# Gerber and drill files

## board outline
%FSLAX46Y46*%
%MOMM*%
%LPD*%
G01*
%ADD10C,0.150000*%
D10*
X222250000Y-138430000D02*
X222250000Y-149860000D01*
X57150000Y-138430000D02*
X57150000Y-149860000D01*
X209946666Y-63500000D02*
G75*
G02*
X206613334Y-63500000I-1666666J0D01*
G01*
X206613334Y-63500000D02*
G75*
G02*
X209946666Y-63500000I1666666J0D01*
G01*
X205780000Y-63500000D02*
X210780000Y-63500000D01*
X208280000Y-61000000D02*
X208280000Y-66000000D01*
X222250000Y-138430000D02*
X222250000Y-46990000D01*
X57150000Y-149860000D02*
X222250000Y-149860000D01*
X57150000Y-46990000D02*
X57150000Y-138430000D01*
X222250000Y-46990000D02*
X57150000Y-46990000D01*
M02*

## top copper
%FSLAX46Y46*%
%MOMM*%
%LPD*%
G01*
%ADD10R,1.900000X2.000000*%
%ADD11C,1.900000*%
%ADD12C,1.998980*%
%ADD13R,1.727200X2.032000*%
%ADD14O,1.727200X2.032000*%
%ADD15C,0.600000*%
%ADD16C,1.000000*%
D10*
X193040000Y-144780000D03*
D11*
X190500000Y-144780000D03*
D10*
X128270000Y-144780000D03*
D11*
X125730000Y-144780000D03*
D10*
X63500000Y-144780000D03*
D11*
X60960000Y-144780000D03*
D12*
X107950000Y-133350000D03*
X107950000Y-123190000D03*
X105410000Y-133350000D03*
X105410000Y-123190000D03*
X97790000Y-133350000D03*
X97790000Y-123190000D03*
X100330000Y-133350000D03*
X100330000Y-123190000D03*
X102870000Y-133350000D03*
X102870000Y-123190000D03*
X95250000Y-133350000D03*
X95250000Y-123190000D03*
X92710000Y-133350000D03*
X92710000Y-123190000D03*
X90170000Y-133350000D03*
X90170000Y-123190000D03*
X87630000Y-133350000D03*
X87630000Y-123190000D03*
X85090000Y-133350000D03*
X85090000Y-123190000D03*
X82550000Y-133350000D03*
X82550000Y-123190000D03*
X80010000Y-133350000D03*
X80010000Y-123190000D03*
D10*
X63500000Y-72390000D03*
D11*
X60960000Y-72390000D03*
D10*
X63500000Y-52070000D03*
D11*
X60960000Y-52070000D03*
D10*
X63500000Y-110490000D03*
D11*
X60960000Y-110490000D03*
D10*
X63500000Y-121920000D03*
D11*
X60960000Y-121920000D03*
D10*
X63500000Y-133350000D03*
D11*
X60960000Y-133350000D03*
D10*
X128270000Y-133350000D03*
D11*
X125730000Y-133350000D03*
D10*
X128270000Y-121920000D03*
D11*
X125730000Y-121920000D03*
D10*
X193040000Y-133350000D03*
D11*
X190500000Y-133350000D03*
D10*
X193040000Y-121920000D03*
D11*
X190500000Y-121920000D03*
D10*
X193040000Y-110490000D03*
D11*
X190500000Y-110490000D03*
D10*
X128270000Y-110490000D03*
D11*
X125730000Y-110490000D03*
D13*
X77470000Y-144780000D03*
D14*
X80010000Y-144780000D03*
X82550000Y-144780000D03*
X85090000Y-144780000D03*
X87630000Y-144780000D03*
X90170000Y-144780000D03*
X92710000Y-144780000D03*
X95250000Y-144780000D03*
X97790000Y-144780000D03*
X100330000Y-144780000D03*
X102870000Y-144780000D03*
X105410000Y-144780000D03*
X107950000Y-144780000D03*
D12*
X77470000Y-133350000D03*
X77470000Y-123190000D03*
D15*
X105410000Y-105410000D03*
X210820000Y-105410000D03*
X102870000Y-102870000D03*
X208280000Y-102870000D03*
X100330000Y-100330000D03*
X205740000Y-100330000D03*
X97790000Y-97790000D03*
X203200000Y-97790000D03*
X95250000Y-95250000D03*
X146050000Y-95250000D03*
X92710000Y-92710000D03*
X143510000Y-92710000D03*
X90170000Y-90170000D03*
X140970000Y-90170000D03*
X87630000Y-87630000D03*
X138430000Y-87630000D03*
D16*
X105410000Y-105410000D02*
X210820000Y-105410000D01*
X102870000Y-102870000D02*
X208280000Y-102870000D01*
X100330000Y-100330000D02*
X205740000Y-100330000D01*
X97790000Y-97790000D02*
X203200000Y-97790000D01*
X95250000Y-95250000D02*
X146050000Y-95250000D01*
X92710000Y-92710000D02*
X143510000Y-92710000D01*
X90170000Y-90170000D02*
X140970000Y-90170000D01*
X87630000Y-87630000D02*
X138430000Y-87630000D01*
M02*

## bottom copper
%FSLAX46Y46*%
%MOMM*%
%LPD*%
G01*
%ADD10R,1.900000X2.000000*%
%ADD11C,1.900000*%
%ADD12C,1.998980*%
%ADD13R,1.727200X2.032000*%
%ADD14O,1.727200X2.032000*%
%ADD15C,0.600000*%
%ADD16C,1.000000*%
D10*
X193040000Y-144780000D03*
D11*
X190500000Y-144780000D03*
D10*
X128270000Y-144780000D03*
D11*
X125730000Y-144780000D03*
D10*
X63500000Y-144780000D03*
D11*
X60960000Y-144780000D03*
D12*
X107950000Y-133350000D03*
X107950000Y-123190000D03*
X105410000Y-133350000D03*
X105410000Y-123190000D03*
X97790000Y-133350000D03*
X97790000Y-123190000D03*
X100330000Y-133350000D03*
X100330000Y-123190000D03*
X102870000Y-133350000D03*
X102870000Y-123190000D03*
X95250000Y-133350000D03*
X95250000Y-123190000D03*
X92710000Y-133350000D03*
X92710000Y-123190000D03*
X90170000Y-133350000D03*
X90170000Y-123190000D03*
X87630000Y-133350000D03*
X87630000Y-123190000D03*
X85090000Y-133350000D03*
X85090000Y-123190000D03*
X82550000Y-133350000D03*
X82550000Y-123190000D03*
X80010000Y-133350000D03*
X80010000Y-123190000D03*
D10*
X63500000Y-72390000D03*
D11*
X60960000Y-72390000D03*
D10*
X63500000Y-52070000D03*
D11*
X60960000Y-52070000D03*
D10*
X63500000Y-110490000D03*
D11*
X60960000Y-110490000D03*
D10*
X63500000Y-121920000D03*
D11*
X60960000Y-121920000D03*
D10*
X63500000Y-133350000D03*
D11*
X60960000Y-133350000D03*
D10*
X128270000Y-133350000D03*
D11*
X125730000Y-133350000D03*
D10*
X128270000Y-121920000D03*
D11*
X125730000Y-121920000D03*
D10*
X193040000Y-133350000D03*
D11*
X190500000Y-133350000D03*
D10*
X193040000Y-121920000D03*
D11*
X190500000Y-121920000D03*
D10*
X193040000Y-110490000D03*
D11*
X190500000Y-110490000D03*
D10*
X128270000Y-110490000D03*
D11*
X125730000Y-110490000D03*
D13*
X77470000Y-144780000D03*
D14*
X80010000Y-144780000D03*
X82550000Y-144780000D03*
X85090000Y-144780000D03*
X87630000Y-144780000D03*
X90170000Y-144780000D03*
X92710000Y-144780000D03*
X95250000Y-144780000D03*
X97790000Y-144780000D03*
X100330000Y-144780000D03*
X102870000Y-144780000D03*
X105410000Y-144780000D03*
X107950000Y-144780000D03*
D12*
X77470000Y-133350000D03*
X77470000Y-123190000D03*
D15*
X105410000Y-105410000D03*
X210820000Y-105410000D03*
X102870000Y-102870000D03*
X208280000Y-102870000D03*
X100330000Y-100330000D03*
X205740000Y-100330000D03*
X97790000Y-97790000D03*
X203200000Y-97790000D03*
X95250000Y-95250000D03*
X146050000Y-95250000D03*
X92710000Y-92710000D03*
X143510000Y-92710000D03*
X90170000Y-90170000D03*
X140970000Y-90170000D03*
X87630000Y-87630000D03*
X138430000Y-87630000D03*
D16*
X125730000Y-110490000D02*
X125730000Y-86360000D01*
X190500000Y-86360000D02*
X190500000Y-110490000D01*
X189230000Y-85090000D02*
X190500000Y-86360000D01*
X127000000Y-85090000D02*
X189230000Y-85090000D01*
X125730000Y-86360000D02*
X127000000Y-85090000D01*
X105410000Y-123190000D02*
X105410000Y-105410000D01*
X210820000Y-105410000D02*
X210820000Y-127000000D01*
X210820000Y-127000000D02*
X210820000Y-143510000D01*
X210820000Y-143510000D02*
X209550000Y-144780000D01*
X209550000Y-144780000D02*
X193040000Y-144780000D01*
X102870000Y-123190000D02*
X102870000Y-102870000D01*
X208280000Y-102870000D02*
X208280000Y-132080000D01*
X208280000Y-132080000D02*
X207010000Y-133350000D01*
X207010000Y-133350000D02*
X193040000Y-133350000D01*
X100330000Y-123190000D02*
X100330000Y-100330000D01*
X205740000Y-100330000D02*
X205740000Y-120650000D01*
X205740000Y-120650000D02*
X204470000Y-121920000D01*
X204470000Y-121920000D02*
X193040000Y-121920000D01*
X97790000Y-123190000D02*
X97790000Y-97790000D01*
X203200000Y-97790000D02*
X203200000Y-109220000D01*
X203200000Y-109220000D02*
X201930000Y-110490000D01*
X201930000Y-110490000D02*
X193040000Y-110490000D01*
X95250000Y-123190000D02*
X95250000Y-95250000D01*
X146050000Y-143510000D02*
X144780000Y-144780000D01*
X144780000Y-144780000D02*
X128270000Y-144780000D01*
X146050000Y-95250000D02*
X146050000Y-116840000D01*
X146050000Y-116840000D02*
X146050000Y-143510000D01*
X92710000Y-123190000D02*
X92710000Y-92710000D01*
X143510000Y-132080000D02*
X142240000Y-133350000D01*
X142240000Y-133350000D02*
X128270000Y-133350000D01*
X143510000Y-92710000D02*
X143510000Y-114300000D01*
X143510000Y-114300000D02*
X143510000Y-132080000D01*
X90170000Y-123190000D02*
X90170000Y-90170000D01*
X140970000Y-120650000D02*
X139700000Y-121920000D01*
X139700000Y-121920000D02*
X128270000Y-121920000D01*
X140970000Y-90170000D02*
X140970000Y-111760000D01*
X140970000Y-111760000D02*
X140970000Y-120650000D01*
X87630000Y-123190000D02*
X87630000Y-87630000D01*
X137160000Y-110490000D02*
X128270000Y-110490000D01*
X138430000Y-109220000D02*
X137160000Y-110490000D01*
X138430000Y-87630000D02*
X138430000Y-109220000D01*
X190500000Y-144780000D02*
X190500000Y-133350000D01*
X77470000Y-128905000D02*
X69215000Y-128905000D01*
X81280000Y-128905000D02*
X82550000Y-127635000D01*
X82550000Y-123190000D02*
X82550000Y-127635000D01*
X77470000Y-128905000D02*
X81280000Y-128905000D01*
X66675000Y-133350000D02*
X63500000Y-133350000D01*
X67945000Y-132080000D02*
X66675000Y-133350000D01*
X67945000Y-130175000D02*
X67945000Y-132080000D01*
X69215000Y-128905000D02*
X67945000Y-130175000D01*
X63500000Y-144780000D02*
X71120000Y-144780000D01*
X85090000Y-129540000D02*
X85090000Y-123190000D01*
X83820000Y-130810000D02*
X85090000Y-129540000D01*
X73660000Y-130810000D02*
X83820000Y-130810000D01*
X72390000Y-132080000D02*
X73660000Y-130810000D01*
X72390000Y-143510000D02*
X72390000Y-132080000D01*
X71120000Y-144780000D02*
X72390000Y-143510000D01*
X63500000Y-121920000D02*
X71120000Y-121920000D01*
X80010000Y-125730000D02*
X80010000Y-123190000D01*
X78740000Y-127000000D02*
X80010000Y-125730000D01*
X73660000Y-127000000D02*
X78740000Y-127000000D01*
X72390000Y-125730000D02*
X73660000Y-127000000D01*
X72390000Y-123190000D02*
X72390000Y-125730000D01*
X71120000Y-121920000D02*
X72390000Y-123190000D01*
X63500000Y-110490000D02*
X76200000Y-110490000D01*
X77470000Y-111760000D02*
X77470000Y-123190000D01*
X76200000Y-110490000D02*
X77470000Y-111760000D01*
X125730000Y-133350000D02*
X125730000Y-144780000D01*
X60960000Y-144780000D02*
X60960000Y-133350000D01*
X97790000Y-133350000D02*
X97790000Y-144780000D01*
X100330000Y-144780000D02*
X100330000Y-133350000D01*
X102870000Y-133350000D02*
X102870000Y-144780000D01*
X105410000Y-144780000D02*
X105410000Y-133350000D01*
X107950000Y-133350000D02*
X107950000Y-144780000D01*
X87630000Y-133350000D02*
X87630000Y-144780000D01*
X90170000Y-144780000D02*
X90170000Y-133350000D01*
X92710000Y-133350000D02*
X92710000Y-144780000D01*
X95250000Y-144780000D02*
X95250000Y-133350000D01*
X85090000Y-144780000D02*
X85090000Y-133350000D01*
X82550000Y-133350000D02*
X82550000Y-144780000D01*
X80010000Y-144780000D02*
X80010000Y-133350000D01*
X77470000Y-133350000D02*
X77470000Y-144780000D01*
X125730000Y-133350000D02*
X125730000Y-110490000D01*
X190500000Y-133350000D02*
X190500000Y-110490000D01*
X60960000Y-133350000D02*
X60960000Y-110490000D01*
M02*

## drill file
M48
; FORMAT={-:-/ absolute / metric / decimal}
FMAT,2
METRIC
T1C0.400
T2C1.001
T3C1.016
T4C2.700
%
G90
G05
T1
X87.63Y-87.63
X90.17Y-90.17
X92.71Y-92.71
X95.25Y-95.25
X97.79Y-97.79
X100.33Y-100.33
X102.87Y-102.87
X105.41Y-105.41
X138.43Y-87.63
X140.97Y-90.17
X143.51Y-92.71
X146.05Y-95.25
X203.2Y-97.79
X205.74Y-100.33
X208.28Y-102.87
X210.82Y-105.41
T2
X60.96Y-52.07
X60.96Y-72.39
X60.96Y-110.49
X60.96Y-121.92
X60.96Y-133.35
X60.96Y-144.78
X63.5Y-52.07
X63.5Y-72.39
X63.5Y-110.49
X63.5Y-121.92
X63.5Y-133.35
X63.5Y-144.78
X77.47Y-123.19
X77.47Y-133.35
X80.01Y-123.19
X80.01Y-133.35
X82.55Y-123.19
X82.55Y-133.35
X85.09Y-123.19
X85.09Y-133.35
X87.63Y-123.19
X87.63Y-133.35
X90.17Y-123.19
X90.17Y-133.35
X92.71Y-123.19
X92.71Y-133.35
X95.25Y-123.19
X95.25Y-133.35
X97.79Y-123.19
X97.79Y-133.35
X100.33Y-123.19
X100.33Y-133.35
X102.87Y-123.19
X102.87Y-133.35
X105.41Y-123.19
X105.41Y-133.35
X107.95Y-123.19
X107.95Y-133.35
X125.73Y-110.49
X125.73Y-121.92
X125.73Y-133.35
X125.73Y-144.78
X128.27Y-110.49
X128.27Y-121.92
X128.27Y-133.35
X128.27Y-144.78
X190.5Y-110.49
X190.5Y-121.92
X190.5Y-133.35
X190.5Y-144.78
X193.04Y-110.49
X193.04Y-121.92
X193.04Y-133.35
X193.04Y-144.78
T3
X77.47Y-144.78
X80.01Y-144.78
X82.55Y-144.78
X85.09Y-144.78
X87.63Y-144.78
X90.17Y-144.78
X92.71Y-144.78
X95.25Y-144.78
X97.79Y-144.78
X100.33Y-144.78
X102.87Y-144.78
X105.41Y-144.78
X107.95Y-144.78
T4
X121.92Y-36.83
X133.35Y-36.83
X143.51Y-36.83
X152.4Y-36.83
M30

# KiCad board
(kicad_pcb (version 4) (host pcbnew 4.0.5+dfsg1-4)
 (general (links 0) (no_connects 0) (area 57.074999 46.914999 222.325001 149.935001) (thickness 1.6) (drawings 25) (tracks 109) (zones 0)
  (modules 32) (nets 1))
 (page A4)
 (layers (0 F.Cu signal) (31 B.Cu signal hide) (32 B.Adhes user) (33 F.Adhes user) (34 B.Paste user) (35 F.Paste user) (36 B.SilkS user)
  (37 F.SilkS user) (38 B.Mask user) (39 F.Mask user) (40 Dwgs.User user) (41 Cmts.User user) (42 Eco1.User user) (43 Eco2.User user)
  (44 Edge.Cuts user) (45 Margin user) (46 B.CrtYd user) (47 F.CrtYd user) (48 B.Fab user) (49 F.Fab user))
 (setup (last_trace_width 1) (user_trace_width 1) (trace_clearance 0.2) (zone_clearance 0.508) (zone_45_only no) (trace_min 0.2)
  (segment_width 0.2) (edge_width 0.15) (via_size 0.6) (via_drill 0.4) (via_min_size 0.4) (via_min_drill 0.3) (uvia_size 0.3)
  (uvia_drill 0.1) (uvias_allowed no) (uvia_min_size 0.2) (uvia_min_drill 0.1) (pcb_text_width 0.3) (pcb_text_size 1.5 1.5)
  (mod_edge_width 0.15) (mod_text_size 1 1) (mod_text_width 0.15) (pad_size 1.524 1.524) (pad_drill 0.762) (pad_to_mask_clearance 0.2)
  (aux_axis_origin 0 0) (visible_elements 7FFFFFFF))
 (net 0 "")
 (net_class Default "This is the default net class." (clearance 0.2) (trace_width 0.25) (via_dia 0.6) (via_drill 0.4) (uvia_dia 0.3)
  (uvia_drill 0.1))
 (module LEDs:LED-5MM (layer F.Cu) (at 193.04 144.78 180)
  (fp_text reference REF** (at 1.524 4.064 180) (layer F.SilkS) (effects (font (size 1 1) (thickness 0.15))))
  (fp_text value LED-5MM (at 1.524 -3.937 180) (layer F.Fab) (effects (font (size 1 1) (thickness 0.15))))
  (pad 1 thru_hole rect (at 0 0 270) (size 2 1.9) (drill 1.00076) (layers *.Cu *.Mask))
  (pad 2 thru_hole circle (at 2.54 0 180) (size 1.9 1.9) (drill 1.00076) (layers *.Cu *.Mask)))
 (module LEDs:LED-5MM (layer F.Cu) (at 128.27 144.78 180)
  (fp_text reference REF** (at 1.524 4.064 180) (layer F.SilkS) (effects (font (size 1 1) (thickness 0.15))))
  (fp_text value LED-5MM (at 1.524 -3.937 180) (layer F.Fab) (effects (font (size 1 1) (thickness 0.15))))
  (pad 1 thru_hole rect (at 0 0 270) (size 2 1.9) (drill 1.00076) (layers *.Cu *.Mask))
  (pad 2 thru_hole circle (at 2.54 0 180) (size 1.9 1.9) (drill 1.00076) (layers *.Cu *.Mask)))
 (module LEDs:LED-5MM (layer F.Cu) (at 63.5 144.78 180)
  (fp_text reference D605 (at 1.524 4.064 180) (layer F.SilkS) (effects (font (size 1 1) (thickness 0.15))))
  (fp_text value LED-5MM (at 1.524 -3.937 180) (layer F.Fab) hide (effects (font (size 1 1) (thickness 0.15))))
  (pad 1 thru_hole rect (at 0 0 270) (size 2 1.9) (drill 1.00076) (layers *.Cu *.Mask))
  (pad 2 thru_hole circle (at 2.54 0 180) (size 1.9 1.9) (drill 1.00076) (layers *.Cu *.Mask)))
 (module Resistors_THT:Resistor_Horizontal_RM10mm (layer F.Cu) (at 107.95 133.35 90)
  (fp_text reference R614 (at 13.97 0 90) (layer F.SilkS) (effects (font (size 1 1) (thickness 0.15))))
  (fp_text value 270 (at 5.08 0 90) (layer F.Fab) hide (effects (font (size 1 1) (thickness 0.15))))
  (pad 1 thru_hole circle (at 0 0 90) (size 1.99898 1.99898) (drill 1.00076) (layers *.Cu *.SilkS *.Mask))
  (pad 2 thru_hole circle (at 10.16 0 90) (size 1.99898 1.99898) (drill 1.00076) (layers *.Cu *.SilkS *.Mask)))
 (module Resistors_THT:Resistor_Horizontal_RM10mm (layer F.Cu) (at 105.41 133.35 90)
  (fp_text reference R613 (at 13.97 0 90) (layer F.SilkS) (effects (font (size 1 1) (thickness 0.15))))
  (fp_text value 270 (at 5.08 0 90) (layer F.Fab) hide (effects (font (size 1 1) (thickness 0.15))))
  (pad 1 thru_hole circle (at 0 0 90) (size 1.99898 1.99898) (drill 1.00076) (layers *.Cu *.SilkS *.Mask))
  (pad 2 thru_hole circle (at 10.16 0 90) (size 1.99898 1.99898) (drill 1.00076) (layers *.Cu *.SilkS *.Mask)))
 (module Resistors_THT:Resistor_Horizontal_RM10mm (layer F.Cu) (at 97.79 133.35 90)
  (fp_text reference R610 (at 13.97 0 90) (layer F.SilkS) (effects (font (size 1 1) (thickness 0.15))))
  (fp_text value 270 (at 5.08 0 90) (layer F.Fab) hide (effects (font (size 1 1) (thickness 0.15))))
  (pad 1 thru_hole circle (at 0 0 90) (size 1.99898 1.99898) (drill 1.00076) (layers *.Cu *.SilkS *.Mask))
  (pad 2 thru_hole circle (at 10.16 0 90) (size 1.99898 1.99898) (drill 1.00076) (layers *.Cu *.SilkS *.Mask)))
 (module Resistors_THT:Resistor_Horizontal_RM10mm (layer F.Cu) (at 100.33 133.35 90)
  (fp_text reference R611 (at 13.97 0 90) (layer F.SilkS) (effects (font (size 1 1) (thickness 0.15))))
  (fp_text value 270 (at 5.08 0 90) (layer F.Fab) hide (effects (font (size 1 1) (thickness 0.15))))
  (pad 1 thru_hole circle (at 0 0 90) (size 1.99898 1.99898) (drill 1.00076) (layers *.Cu *.SilkS *.Mask))
  (pad 2 thru_hole circle (at 10.16 0 90) (size 1.99898 1.99898) (drill 1.00076) (layers *.Cu *.SilkS *.Mask)))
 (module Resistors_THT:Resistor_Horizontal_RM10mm (layer F.Cu) (at 102.87 133.35 90)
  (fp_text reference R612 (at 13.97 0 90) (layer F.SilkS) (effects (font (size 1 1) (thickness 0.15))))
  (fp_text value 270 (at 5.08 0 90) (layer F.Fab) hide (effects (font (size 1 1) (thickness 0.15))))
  (pad 1 thru_hole circle (at 0 0 90) (size 1.99898 1.99898) (drill 1.00076) (layers *.Cu *.SilkS *.Mask))
  (pad 2 thru_hole circle (at 10.16 0 90) (size 1.99898 1.99898) (drill 1.00076) (layers *.Cu *.SilkS *.Mask)))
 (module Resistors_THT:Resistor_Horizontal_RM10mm (layer F.Cu) (at 95.25 133.35 90)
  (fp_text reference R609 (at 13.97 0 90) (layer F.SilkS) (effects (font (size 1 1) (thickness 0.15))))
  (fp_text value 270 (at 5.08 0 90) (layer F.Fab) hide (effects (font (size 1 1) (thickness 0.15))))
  (pad 1 thru_hole circle (at 0 0 90) (size 1.99898 1.99898) (drill 1.00076) (layers *.Cu *.SilkS *.Mask))
  (pad 2 thru_hole circle (at 10.16 0 90) (size 1.99898 1.99898) (drill 1.00076) (layers *.Cu *.SilkS *.Mask)))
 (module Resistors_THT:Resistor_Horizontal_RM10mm (layer F.Cu) (at 92.71 133.35 90)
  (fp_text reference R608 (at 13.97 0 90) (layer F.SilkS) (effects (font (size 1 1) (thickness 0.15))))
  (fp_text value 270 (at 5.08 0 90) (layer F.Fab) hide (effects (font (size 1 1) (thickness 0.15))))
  (pad 1 thru_hole circle (at 0 0 90) (size 1.99898 1.99898) (drill 1.00076) (layers *.Cu *.SilkS *.Mask))
  (pad 2 thru_hole circle (at 10.16 0 90) (size 1.99898 1.99898) (drill 1.00076) (layers *.Cu *.SilkS *.Mask)))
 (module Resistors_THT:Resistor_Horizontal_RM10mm (layer F.Cu) (at 90.17 133.35 90)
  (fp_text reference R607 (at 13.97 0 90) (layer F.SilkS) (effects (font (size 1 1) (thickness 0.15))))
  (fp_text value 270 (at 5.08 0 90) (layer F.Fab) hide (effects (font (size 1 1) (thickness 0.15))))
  (pad 1 thru_hole circle (at 0 0 90) (size 1.99898 1.99898) (drill 1.00076) (layers *.Cu *.SilkS *.Mask))
  (pad 2 thru_hole circle (at 10.16 0 90) (size 1.99898 1.99898) (drill 1.00076) (layers *.Cu *.SilkS *.Mask)))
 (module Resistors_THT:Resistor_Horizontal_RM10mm (layer F.Cu) (at 87.63 133.35 90)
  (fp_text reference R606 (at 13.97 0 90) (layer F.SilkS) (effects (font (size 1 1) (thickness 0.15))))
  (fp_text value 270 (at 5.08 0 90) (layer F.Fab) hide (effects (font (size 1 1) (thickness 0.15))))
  (pad 1 thru_hole circle (at 0 0 90) (size 1.99898 1.99898) (drill 1.00076) (layers *.Cu *.SilkS *.Mask))
  (pad 2 thru_hole circle (at 10.16 0 90) (size 1.99898 1.99898) (drill 1.00076) (layers *.Cu *.SilkS *.Mask)))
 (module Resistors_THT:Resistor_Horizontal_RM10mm (layer F.Cu) (at 85.09 133.35 90)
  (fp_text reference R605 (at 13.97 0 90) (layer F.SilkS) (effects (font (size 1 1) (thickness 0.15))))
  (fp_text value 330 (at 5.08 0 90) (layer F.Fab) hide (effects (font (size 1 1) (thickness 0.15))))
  (pad 1 thru_hole circle (at 0 0 90) (size 1.99898 1.99898) (drill 1.00076) (layers *.Cu *.SilkS *.Mask))
  (pad 2 thru_hole circle (at 10.16 0 90) (size 1.99898 1.99898) (drill 1.00076) (layers *.Cu *.SilkS *.Mask)))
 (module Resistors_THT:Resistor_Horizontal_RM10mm (layer F.Cu) (at 82.55 133.35 90)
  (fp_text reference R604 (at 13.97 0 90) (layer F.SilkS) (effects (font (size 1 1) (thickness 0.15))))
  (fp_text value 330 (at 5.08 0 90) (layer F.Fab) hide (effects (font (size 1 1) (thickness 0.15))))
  (pad 1 thru_hole circle (at 0 0 90) (size 1.99898 1.99898) (drill 1.00076) (layers *.Cu *.SilkS *.Mask))
  (pad 2 thru_hole circle (at 10.16 0 90) (size 1.99898 1.99898) (drill 1.00076) (layers *.Cu *.SilkS *.Mask)))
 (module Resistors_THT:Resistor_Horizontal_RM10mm (layer F.Cu) (at 80.01 133.35 90)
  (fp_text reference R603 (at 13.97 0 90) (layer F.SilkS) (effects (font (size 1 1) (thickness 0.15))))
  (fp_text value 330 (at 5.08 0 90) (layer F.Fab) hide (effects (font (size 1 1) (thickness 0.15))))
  (pad 1 thru_hole circle (at 0 0 90) (size 1.99898 1.99898) (drill 1.00076) (layers *.Cu *.SilkS *.Mask))
  (pad 2 thru_hole circle (at 10.16 0 90) (size 1.99898 1.99898) (drill 1.00076) (layers *.Cu *.SilkS *.Mask)))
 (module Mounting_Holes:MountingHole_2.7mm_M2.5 (layer F.Cu) (at 152.4 36.83)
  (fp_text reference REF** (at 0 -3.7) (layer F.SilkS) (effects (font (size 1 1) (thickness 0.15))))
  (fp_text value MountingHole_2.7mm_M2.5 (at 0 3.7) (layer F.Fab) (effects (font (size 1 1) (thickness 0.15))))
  (pad 1 np_thru_hole circle (at 0 0) (size 2.7 2.7) (drill 2.7) (layers *.Cu *.Mask)))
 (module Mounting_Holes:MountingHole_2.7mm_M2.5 (layer F.Cu) (at 143.51 36.83)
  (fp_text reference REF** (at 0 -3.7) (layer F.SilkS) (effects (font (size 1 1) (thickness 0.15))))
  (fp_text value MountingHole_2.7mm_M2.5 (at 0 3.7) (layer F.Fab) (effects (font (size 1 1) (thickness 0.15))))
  (pad 1 np_thru_hole circle (at 0 0) (size 2.7 2.7) (drill 2.7) (layers *.Cu *.Mask)))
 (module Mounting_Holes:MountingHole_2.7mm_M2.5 (layer F.Cu) (at 133.35 36.83)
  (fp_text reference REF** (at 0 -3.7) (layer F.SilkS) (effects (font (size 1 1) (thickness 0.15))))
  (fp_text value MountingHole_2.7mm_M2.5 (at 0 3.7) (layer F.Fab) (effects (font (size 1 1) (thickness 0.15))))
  (pad 1 np_thru_hole circle (at 0 0) (size 2.7 2.7) (drill 2.7) (layers *.Cu *.Mask)))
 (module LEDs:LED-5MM (layer F.Cu) (at 63.5 72.39 180)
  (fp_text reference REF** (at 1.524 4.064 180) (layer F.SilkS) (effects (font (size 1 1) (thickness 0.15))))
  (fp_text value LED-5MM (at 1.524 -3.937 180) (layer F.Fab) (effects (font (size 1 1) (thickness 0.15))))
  (pad 1 thru_hole rect (at 0 0 270) (size 2 1.9) (drill 1.00076) (layers *.Cu *.Mask))
  (pad 2 thru_hole circle (at 2.54 0 180) (size 1.9 1.9) (drill 1.00076) (layers *.Cu *.Mask)))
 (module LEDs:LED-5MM (layer F.Cu) (at 63.5 52.07 180)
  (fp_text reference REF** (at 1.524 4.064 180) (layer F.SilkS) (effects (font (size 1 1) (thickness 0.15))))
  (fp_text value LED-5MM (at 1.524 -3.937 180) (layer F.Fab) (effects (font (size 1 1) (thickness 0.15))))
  (pad 1 thru_hole rect (at 0 0 270) (size 2 1.9) (drill 1.00076) (layers *.Cu *.Mask))
  (pad 2 thru_hole circle (at 2.54 0 180) (size 1.9 1.9) (drill 1.00076) (layers *.Cu *.Mask)))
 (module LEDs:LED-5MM (layer F.Cu) (at 63.5 110.49 180)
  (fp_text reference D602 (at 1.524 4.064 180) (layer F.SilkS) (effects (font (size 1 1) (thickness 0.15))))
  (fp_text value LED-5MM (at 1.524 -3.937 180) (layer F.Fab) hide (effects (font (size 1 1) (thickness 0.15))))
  (pad 1 thru_hole rect (at 0 0 270) (size 2 1.9) (drill 1.00076) (layers *.Cu *.Mask))
  (pad 2 thru_hole circle (at 2.54 0 180) (size 1.9 1.9) (drill 1.00076) (layers *.Cu *.Mask)))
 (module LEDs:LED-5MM (layer F.Cu) (at 63.5 121.92 180)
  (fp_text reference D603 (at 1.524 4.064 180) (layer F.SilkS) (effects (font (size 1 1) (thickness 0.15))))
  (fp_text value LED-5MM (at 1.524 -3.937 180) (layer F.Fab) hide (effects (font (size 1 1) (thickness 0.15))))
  (pad 1 thru_hole rect (at 0 0 270) (size 2 1.9) (drill 1.00076) (layers *.Cu *.Mask))
  (pad 2 thru_hole circle (at 2.54 0 180) (size 1.9 1.9) (drill 1.00076) (layers *.Cu *.Mask)))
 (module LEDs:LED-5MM (layer F.Cu) (at 63.5 133.35 180)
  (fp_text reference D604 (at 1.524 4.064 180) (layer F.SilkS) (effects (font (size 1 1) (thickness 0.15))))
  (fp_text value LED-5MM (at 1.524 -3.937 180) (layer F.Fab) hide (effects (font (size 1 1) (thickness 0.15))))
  (pad 1 thru_hole rect (at 0 0 270) (size 2 1.9) (drill 1.00076) (layers *.Cu *.Mask))
  (pad 2 thru_hole circle (at 2.54 0 180) (size 1.9 1.9) (drill 1.00076) (layers *.Cu *.Mask)))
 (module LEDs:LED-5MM (layer F.Cu) (at 128.27 133.35 180)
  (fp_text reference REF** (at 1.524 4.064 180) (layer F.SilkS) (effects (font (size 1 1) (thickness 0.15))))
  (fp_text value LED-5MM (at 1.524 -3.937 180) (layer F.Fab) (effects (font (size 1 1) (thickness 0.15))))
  (pad 1 thru_hole rect (at 0 0 270) (size 2 1.9) (drill 1.00076) (layers *.Cu *.Mask))
  (pad 2 thru_hole circle (at 2.54 0 180) (size 1.9 1.9) (drill 1.00076) (layers *.Cu *.Mask)))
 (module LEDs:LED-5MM (layer F.Cu) (at 128.27 121.92 180)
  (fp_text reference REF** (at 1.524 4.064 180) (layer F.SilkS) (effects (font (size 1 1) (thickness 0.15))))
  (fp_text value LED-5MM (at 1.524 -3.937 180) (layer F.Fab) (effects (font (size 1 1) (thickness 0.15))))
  (pad 1 thru_hole rect (at 0 0 270) (size 2 1.9) (drill 1.00076) (layers *.Cu *.Mask))
  (pad 2 thru_hole circle (at 2.54 0 180) (size 1.9 1.9) (drill 1.00076) (layers *.Cu *.Mask)))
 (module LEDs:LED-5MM (layer F.Cu) (at 193.04 133.35 180)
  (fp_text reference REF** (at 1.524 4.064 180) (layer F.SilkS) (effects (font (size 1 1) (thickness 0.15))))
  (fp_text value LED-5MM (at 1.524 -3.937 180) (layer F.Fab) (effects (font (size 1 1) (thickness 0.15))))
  (pad 1 thru_hole rect (at 0 0 270) (size 2 1.9) (drill 1.00076) (layers *.Cu *.Mask))
  (pad 2 thru_hole circle (at 2.54 0 180) (size 1.9 1.9) (drill 1.00076) (layers *.Cu *.Mask)))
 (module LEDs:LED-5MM (layer F.Cu) (at 193.04 121.92 180)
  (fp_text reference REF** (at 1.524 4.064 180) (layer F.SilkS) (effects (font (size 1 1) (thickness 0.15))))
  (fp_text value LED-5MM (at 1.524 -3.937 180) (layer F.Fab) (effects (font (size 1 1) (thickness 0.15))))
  (pad 1 thru_hole rect (at 0 0 270) (size 2 1.9) (drill 1.00076) (layers *.Cu *.Mask))
  (pad 2 thru_hole circle (at 2.54 0 180) (size 1.9 1.9) (drill 1.00076) (layers *.Cu *.Mask)))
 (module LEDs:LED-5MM (layer F.Cu) (at 193.04 110.49 180)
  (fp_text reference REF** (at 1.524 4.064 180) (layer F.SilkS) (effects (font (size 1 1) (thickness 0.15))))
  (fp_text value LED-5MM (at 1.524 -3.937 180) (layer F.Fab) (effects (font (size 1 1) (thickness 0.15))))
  (pad 1 thru_hole rect (at 0 0 270) (size 2 1.9) (drill 1.00076) (layers *.Cu *.Mask))
  (pad 2 thru_hole circle (at 2.54 0 180) (size 1.9 1.9) (drill 1.00076) (layers *.Cu *.Mask)))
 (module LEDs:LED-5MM (layer F.Cu) (at 128.27 110.49 180)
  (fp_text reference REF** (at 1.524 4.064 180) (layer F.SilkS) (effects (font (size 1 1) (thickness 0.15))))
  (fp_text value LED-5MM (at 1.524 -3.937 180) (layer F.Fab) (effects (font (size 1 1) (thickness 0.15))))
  (pad 1 thru_hole rect (at 0 0 270) (size 2 1.9) (drill 1.00076) (layers *.Cu *.Mask))
  (pad 2 thru_hole circle (at 2.54 0 180) (size 1.9 1.9) (drill 1.00076) (layers *.Cu *.Mask)))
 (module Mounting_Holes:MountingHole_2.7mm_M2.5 (layer F.Cu) (at 121.92 36.83)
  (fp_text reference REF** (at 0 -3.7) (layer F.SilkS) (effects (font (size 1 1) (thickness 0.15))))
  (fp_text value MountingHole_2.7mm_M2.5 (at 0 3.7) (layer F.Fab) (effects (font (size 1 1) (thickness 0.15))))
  (pad 1 np_thru_hole circle (at 0 0) (size 2.7 2.7) (drill 2.7) (layers *.Cu *.Mask)))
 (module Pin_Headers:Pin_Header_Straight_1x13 (layer F.Cu) (at 77.47 144.78 90)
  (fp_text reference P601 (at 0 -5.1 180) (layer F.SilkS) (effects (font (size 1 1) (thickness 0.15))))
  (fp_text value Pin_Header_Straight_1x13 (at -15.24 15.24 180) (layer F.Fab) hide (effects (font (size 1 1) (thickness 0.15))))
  (pad 1 thru_hole rect (at 0 0 90) (size 2.032 1.7272) (drill 1.016) (layers *.Cu *.Mask))
  (pad 2 thru_hole oval (at 0 2.54 90) (size 2.032 1.7272) (drill 1.016) (layers *.Cu *.Mask))
  (pad 3 thru_hole oval (at 0 5.08 90) (size 2.032 1.7272) (drill 1.016) (layers *.Cu *.Mask))
  (pad 4 thru_hole oval (at 0 7.62 90) (size 2.032 1.7272) (drill 1.016) (layers *.Cu *.Mask))
  (pad 5 thru_hole oval (at 0 10.16 90) (size 2.032 1.7272) (drill 1.016) (layers *.Cu *.Mask))
  (pad 6 thru_hole oval (at 0 12.7 90) (size 2.032 1.7272) (drill 1.016) (layers *.Cu *.Mask))
  (pad 7 thru_hole oval (at 0 15.24 90) (size 2.032 1.7272) (drill 1.016) (layers *.Cu *.Mask))
  (pad 8 thru_hole oval (at 0 17.78 90) (size 2.032 1.7272) (drill 1.016) (layers *.Cu *.Mask))
  (pad 9 thru_hole oval (at 0 20.32 90) (size 2.032 1.7272) (drill 1.016) (layers *.Cu *.Mask))
  (pad 10 thru_hole oval (at 0 22.86 90) (size 2.032 1.7272) (drill 1.016) (layers *.Cu *.Mask))
  (pad 11 thru_hole oval (at 0 25.4 90) (size 2.032 1.7272) (drill 1.016) (layers *.Cu *.Mask))
  (pad 12 thru_hole oval (at 0 27.94 90) (size 2.032 1.7272) (drill 1.016) (layers *.Cu *.Mask))
  (pad 13 thru_hole oval (at 0 30.48 90) (size 2.032 1.7272) (drill 1.016) (layers *.Cu *.Mask)))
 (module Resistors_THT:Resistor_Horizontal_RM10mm (layer F.Cu) (at 77.47 133.35 90)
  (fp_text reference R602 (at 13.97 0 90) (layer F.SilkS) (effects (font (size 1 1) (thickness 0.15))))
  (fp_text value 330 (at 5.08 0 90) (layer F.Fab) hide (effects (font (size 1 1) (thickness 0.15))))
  (pad 1 thru_hole circle (at 0 0 90) (size 1.99898 1.99898) (drill 1.00076) (layers *.Cu *.SilkS *.Mask))
  (pad 2 thru_hole circle (at 10.16 0 90) (size 1.99898 1.99898) (drill 1.00076) (layers *.Cu *.SilkS *.Mask)))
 (gr_line (start 222.25 138.43) (end 222.25 149.86) (angle 90) (layer Edge.Cuts) (width 0.15))
 (gr_line (start 57.15 138.43) (end 57.15 149.86) (angle 90) (layer Edge.Cuts) (width 0.15))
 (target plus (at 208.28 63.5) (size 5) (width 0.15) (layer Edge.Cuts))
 (gr_line (start 222.25 138.43) (end 222.25 46.99) (angle 90) (layer Edge.Cuts) (width 0.15))
 (gr_line (start 57.15 149.86) (end 222.25 149.86) (angle 90) (layer Edge.Cuts) (width 0.15))
 (gr_line (start 57.15 46.99) (end 57.15 138.43) (angle 90) (layer Edge.Cuts) (width 0.15))
 (gr_line (start 222.25 46.99) (end 57.15 46.99) (angle 90) (layer Edge.Cuts) (width 0.15))
 (segment (start 125.73 110.49) (end 125.73 86.36) (width 1) (layer B.Cu) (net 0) (status 400000))
 (segment (start 190.5 86.36) (end 190.5 110.49) (width 1) (layer B.Cu) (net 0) (status 800000))
 (segment (start 189.23 85.09) (end 190.5 86.36) (width 1) (layer B.Cu) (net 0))
 (segment (start 127 85.09) (end 189.23 85.09) (width 1) (layer B.Cu) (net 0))
 (segment (start 125.73 86.36) (end 127 85.09) (width 1) (layer B.Cu) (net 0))
 (via (at 105.41 105.41) (size 0.6) (drill 0.4) (layers F.Cu B.Cu) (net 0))
 (segment (start 105.41 123.19) (end 105.41 105.41) (width 1) (layer B.Cu) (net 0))
 (via (at 210.82 105.41) (size 0.6) (drill 0.4) (layers F.Cu B.Cu) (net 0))
 (segment (start 210.82 105.41) (end 210.82 127) (width 1) (layer B.Cu) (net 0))
 (segment (start 210.82 127) (end 210.82 143.51) (width 1) (layer B.Cu) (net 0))
 (segment (start 210.82 143.51) (end 209.55 144.78) (width 1) (layer B.Cu) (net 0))
 (segment (start 209.55 144.78) (end 193.04 144.78) (width 1) (layer B.Cu) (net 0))
 (segment (start 105.41 105.41) (end 210.82 105.41) (width 1) (layer F.Cu) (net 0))
 (via (at 102.87 102.87) (size 0.6) (drill 0.4) (layers F.Cu B.Cu) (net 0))
 (segment (start 102.87 123.19) (end 102.87 102.87) (width 1) (layer B.Cu) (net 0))
 (via (at 208.28 102.87) (size 0.6) (drill 0.4) (layers F.Cu B.Cu) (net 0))
 (segment (start 208.28 102.87) (end 208.28 132.08) (width 1) (layer B.Cu) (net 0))
 (segment (start 208.28 132.08) (end 207.01 133.35) (width 1) (layer B.Cu) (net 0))
 (segment (start 207.01 133.35) (end 193.04 133.35) (width 1) (layer B.Cu) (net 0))
 (segment (start 102.87 102.87) (end 208.28 102.87) (width 1) (layer F.Cu) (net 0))
 (via (at 100.33 100.33) (size 0.6) (drill 0.4) (layers F.Cu B.Cu) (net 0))
 (segment (start 100.33 123.19) (end 100.33 100.33) (width 1) (layer B.Cu) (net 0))
 (via (at 205.74 100.33) (size 0.6) (drill 0.4) (layers F.Cu B.Cu) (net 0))
 (segment (start 205.74 100.33) (end 205.74 120.65) (width 1) (layer B.Cu) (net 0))
 (segment (start 205.74 120.65) (end 204.47 121.92) (width 1) (layer B.Cu) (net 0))
 (segment (start 204.47 121.92) (end 193.04 121.92) (width 1) (layer B.Cu) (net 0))
 (segment (start 100.33 100.33) (end 205.74 100.33) (width 1) (layer F.Cu) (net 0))
 (via (at 97.79 97.79) (size 0.6) (drill 0.4) (layers F.Cu B.Cu) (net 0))
 (segment (start 97.79 123.19) (end 97.79 97.79) (width 1) (layer B.Cu) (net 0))
 (via (at 203.2 97.79) (size 0.6) (drill 0.4) (layers F.Cu B.Cu) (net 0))
 (segment (start 203.2 97.79) (end 203.2 109.22) (width 1) (layer B.Cu) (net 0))
 (segment (start 203.2 109.22) (end 201.93 110.49) (width 1) (layer B.Cu) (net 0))
 (segment (start 201.93 110.49) (end 193.04 110.49) (width 1) (layer B.Cu) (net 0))
 (segment (start 97.79 97.79) (end 203.2 97.79) (width 1) (layer F.Cu) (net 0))
 (via (at 95.25 95.25) (size 0.6) (drill 0.4) (layers F.Cu B.Cu) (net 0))
 (segment (start 95.25 123.19) (end 95.25 95.25) (width 1) (layer B.Cu) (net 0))
 (segment (start 146.05 143.51) (end 144.78 144.78) (width 1) (layer B.Cu) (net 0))
 (segment (start 144.78 144.78) (end 128.27 144.78) (width 1) (layer B.Cu) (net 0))
 (segment (start 95.25 95.25) (end 146.05 95.25) (width 1) (layer F.Cu) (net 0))
 (via (at 146.05 95.25) (size 0.6) (drill 0.4) (layers F.Cu B.Cu) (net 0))
 (segment (start 146.05 95.25) (end 146.05 116.84) (width 1) (layer B.Cu) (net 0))
 (segment (start 146.05 116.84) (end 146.05 143.51) (width 1) (layer B.Cu) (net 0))
 (via (at 92.71 92.71) (size 0.6) (drill 0.4) (layers F.Cu B.Cu) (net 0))
 (segment (start 92.71 123.19) (end 92.71 92.71) (width 1) (layer B.Cu) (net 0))
 (segment (start 143.51 132.08) (end 142.24 133.35) (width 1) (layer B.Cu) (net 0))
 (segment (start 142.24 133.35) (end 128.27 133.35) (width 1) (layer B.Cu) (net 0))
 (segment (start 143.51 92.71) (end 143.51 114.3) (width 1) (layer B.Cu) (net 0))
 (via (at 143.51 92.71) (size 0.6) (drill 0.4) (layers F.Cu B.Cu) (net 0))
 (segment (start 92.71 92.71) (end 143.51 92.71) (width 1) (layer F.Cu) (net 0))
 (segment (start 143.51 114.3) (end 143.51 132.08) (width 1) (layer B.Cu) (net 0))
 (via (at 90.17 90.17) (size 0.6) (drill 0.4) (layers F.Cu B.Cu) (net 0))
 (segment (start 90.17 123.19) (end 90.17 90.17) (width 1) (layer B.Cu) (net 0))
 (segment (start 140.97 120.65) (end 139.7 121.92) (width 1) (layer B.Cu) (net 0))
 (segment (start 139.7 121.92) (end 128.27 121.92) (width 1) (layer B.Cu) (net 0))
 (segment (start 140.97 90.17) (end 140.97 111.76) (width 1) (layer B.Cu) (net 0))
 (via (at 140.97 90.17) (size 0.6) (drill 0.4) (layers F.Cu B.Cu) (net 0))
 (segment (start 90.17 90.17) (end 140.97 90.17) (width 1) (layer F.Cu) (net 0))
 (segment (start 140.97 111.76) (end 140.97 120.65) (width 1) (layer B.Cu) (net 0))
 (via (at 87.63 87.63) (size 0.6) (drill 0.4) (layers F.Cu B.Cu) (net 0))
 (segment (start 87.63 123.19) (end 87.63 87.63) (width 1) (layer B.Cu) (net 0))
 (segment (start 137.16 110.49) (end 128.27 110.49) (width 1) (layer B.Cu) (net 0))
 (segment (start 138.43 109.22) (end 137.16 110.49) (width 1) (layer B.Cu) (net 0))
 (segment (start 138.43 87.63) (end 138.43 109.22) (width 1) (layer B.Cu) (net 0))
 (via (at 138.43 87.63) (size 0.6) (drill 0.4) (layers F.Cu B.Cu) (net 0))
 (segment (start 87.63 87.63) (end 138.43 87.63) (width 1) (layer F.Cu) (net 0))
 (segment (start 190.5 144.78) (end 190.5 133.35) (width 1) (layer B.Cu) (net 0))
 (segment (start 77.47 128.905) (end 69.215 128.905) (width 1) (layer B.Cu) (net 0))
 (segment (start 81.28 128.905) (end 82.55 127.635) (width 1) (layer B.Cu) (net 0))
 (segment (start 82.55 123.19) (end 82.55 127.635) (width 1) (layer B.Cu) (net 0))
 (segment (start 77.47 128.905) (end 81.28 128.905) (width 1) (layer B.Cu) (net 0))
 (segment (start 66.675 133.35) (end 63.5 133.35) (width 1) (layer B.Cu) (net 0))
 (segment (start 67.945 132.08) (end 66.675 133.35) (width 1) (layer B.Cu) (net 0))
 (segment (start 67.945 130.175) (end 67.945 132.08) (width 1) (layer B.Cu) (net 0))
 (segment (start 69.215 128.905) (end 67.945 130.175) (width 1) (layer B.Cu) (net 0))
 (segment (start 63.5 144.78) (end 71.12 144.78) (width 1) (layer B.Cu) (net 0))
 (segment (start 85.09 129.54) (end 85.09 123.19) (width 1) (layer B.Cu) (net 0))
 (segment (start 83.82 130.81) (end 85.09 129.54) (width 1) (layer B.Cu) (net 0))
 (segment (start 73.66 130.81) (end 83.82 130.81) (width 1) (layer B.Cu) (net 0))
 (segment (start 72.39 132.08) (end 73.66 130.81) (width 1) (layer B.Cu) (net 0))
 (segment (start 72.39 143.51) (end 72.39 132.08) (width 1) (layer B.Cu) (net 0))
 (segment (start 71.12 144.78) (end 72.39 143.51) (width 1) (layer B.Cu) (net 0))
 (segment (start 63.5 121.92) (end 71.12 121.92) (width 1) (layer B.Cu) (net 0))
 (segment (start 80.01 125.73) (end 80.01 123.19) (width 1) (layer B.Cu) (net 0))
 (segment (start 78.74 127) (end 80.01 125.73) (width 1) (layer B.Cu) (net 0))
 (segment (start 73.66 127) (end 78.74 127) (width 1) (layer B.Cu) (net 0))
 (segment (start 72.39 125.73) (end 73.66 127) (width 1) (layer B.Cu) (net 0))
 (segment (start 72.39 123.19) (end 72.39 125.73) (width 1) (layer B.Cu) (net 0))
 (segment (start 71.12 121.92) (end 72.39 123.19) (width 1) (layer B.Cu) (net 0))
 (segment (start 63.5 110.49) (end 76.2 110.49) (width 1) (layer B.Cu) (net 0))
 (segment (start 77.47 111.76) (end 77.47 123.19) (width 1) (layer B.Cu) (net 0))
 (segment (start 76.2 110.49) (end 77.47 111.76) (width 1) (layer B.Cu) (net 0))
 (segment (start 125.73 133.35) (end 125.73 144.78) (width 1) (layer B.Cu) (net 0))
 (segment (start 60.96 144.78) (end 60.96 133.35) (width 1) (layer B.Cu) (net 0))
 (segment (start 97.79 133.35) (end 97.79 144.78) (width 1) (layer B.Cu) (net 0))
 (segment (start 100.33 144.78) (end 100.33 133.35) (width 1) (layer B.Cu) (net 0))
 (segment (start 102.87 133.35) (end 102.87 144.78) (width 1) (layer B.Cu) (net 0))
 (segment (start 105.41 144.78) (end 105.41 133.35) (width 1) (layer B.Cu) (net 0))
 (segment (start 107.95 133.35) (end 107.95 144.78) (width 1) (layer B.Cu) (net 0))
 (segment (start 87.63 133.35) (end 87.63 144.78) (width 1) (layer B.Cu) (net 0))
 (segment (start 90.17 144.78) (end 90.17 133.35) (width 1) (layer B.Cu) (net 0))
 (segment (start 92.71 133.35) (end 92.71 144.78) (width 1) (layer B.Cu) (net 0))
 (segment (start 95.25 144.78) (end 95.25 133.35) (width 1) (layer B.Cu) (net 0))
 (segment (start 85.09 144.78) (end 85.09 133.35) (width 1) (layer B.Cu) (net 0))
 (segment (start 82.55 133.35) (end 82.55 144.78) (width 1) (layer B.Cu) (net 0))
 (segment (start 80.01 144.78) (end 80.01 133.35) (width 1) (layer B.Cu) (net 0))
 (segment (start 77.47 133.35) (end 77.47 144.78) (width 1) (layer B.Cu) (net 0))
 (segment (start 125.73 133.35) (end 125.73 110.49) (width 1) (layer B.Cu) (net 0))
 (segment (start 190.5 133.35) (end 190.5 110.49) (width 1) (layer B.Cu) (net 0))
 (segment (start 60.96 133.35) (end 60.96 110.49) (width 1) (layer B.Cu) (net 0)))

